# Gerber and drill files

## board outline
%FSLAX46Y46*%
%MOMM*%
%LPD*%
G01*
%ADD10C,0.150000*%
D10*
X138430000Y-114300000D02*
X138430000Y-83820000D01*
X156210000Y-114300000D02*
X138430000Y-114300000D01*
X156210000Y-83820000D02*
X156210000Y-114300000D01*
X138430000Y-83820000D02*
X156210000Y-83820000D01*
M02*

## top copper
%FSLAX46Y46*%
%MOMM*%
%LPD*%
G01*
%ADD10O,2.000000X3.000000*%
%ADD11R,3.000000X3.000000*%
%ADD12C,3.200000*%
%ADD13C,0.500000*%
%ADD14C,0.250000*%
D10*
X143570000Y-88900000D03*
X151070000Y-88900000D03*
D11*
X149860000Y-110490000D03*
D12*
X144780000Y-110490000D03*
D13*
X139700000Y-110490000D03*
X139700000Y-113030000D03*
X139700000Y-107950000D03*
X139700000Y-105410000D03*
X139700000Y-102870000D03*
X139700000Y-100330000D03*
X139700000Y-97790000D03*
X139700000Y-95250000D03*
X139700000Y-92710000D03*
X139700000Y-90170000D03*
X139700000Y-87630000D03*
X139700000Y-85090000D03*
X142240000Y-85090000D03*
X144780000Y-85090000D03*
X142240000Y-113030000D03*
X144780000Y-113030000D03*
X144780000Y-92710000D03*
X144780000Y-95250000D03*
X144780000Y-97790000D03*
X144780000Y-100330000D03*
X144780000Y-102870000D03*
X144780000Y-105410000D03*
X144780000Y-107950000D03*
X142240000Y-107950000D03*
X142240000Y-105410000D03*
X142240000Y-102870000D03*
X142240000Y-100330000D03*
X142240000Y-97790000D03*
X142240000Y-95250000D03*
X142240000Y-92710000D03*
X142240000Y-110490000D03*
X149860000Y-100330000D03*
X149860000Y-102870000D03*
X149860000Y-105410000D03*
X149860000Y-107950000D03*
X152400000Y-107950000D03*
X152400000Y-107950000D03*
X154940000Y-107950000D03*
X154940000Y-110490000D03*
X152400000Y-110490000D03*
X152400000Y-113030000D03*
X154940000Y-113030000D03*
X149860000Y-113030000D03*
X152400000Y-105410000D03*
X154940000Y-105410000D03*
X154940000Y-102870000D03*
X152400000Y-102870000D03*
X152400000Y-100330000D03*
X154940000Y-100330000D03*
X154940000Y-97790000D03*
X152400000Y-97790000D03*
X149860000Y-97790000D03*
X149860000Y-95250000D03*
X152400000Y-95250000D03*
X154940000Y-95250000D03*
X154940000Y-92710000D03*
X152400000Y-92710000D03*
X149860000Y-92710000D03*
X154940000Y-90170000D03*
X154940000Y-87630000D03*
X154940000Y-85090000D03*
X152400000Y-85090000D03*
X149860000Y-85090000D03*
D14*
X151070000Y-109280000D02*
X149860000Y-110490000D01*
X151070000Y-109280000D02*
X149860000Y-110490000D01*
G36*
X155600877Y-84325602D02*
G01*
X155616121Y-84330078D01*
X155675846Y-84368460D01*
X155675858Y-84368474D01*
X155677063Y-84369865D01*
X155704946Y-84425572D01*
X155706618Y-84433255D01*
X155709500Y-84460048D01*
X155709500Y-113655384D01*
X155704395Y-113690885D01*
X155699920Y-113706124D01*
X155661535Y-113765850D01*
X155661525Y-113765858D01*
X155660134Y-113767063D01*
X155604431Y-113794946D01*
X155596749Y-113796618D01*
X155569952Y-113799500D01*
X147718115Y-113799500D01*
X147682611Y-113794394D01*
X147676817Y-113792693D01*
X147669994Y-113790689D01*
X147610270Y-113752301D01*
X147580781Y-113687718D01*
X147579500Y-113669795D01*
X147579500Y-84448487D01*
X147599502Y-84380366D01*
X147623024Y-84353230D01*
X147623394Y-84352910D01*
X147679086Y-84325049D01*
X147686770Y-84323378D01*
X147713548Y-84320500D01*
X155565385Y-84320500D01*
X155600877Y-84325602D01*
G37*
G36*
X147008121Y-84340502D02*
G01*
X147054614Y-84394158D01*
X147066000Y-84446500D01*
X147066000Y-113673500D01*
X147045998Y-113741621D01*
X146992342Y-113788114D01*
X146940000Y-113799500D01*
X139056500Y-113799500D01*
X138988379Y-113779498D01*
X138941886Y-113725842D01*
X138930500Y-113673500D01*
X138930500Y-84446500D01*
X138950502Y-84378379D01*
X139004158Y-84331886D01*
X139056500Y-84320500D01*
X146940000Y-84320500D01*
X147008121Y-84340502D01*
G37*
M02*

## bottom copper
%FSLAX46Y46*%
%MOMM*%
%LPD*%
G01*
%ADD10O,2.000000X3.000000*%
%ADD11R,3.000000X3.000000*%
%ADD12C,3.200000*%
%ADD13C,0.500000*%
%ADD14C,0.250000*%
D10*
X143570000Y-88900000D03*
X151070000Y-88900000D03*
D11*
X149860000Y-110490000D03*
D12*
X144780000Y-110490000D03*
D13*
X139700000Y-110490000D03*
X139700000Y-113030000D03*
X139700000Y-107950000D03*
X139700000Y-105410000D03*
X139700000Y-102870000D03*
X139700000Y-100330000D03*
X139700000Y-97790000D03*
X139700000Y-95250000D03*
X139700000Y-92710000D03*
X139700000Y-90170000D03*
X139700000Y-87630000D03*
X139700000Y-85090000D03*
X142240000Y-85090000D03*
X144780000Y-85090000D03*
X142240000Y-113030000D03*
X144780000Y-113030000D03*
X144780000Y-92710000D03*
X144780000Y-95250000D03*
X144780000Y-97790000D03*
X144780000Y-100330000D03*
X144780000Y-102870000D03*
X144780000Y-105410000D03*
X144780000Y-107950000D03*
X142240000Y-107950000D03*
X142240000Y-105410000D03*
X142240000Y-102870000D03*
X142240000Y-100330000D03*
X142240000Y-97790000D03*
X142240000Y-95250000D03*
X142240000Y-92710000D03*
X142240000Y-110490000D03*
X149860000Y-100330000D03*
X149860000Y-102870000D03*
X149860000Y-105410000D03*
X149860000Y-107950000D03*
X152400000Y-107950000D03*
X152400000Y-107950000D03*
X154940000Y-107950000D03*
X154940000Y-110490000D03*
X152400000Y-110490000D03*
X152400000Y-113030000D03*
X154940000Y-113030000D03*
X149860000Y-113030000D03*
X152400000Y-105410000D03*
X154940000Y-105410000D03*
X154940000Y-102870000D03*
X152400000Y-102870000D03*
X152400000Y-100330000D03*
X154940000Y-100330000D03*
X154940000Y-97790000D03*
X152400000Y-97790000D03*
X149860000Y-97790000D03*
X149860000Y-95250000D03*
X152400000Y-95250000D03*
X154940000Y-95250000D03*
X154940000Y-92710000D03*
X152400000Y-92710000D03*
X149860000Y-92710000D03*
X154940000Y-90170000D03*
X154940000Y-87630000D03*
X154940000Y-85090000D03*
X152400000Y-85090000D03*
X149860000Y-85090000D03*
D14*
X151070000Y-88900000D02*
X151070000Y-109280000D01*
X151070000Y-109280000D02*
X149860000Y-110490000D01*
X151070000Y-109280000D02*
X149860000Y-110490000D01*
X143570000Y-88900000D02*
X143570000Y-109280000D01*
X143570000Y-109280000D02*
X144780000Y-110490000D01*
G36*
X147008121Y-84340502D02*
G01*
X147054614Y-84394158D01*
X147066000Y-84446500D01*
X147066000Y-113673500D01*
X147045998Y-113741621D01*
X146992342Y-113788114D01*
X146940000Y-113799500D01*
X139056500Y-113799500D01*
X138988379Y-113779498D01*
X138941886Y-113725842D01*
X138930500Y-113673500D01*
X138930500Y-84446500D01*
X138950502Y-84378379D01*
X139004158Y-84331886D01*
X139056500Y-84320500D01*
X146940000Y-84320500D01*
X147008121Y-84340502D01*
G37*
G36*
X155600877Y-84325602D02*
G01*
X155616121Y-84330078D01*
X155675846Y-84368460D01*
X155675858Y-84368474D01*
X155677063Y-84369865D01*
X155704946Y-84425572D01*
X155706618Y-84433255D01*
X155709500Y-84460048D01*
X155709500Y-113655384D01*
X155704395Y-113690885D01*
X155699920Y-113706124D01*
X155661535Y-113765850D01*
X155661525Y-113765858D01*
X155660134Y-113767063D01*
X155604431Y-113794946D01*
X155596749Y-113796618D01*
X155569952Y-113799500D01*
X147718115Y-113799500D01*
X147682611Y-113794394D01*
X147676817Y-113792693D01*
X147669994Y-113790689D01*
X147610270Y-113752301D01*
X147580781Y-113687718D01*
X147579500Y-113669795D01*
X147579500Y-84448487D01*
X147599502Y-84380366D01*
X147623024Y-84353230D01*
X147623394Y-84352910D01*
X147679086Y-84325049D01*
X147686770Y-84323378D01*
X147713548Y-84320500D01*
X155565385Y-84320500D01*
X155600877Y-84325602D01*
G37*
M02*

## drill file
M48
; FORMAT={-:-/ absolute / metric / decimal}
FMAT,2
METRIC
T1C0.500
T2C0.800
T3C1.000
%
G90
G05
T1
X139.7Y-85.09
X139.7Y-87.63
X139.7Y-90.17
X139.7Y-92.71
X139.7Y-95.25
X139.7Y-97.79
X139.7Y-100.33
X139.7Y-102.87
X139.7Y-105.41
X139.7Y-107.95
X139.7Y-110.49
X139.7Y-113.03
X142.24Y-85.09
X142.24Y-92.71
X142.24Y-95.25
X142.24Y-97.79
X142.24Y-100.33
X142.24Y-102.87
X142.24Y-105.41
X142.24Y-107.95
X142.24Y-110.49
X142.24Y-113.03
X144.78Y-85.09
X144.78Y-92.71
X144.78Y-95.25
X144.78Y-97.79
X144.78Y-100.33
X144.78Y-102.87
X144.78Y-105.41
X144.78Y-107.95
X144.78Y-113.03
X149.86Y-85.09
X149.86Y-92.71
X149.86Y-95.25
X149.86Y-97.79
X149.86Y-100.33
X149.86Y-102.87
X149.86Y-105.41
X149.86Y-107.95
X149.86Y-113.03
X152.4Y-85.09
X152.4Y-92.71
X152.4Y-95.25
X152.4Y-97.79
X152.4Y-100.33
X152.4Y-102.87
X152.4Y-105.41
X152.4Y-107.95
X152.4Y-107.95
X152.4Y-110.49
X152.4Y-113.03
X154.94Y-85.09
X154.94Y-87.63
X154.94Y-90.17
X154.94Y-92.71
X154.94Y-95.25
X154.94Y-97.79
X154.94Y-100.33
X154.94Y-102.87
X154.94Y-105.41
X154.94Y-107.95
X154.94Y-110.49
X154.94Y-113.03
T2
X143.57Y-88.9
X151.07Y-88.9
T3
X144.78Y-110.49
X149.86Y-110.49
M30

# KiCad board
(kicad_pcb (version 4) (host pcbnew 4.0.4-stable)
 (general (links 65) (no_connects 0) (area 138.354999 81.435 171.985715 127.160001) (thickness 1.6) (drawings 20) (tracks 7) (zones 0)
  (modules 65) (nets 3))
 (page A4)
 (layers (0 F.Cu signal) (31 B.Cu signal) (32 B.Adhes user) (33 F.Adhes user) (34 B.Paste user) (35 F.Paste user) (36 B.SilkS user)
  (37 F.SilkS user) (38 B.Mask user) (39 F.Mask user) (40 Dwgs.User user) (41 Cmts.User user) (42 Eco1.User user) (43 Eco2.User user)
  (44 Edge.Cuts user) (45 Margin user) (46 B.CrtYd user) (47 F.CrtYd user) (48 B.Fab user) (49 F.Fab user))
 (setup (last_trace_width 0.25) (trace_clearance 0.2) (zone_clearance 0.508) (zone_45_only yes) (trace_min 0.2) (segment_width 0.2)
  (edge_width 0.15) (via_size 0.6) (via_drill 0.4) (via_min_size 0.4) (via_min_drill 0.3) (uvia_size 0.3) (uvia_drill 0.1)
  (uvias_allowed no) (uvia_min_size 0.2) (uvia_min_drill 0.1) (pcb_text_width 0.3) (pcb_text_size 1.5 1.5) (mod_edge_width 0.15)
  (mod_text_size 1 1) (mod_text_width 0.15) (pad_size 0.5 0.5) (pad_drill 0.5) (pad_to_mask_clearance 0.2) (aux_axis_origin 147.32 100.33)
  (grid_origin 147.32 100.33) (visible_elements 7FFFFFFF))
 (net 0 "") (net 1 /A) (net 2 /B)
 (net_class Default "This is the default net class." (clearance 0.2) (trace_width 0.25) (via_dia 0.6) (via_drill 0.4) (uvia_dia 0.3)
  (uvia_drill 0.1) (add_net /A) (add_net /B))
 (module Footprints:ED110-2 (layer F.Cu) (at 147.32 88.9)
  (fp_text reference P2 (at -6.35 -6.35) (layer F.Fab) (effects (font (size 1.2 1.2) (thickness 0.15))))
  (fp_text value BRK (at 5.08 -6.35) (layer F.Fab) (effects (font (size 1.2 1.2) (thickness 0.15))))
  (pad 1 thru_hole oval (at -3.75 0) (size 2 3) (drill 0.8) (layers *.Cu *.Mask) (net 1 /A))
  (pad 2 thru_hole oval (at 3.75 0) (size 2 3) (drill 0.8) (layers *.Cu *.Mask) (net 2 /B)))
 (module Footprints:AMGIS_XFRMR (layer F.Cu) (at 147.32 110.49 180)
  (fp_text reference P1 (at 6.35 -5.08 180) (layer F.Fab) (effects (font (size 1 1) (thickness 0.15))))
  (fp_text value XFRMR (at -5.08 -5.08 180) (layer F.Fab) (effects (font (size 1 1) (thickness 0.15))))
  (pad 1 thru_hole rect (at -2.54 0 180) (size 3 3) (drill 1) (layers *.Cu *.Mask) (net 2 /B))
  (pad 2 thru_hole circle (at 2.54 0 180) (size 3.2 3.2) (drill 1) (layers *.Cu *.Mask) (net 1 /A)))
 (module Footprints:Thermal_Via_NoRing (layer F.Cu) (at 139.7 110.49)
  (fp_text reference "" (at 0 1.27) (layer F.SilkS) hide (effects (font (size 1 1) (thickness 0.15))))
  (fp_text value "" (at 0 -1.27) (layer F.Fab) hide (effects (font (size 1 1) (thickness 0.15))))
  (pad "" thru_hole circle (at 0 0) (size 0.5 0.5) (drill 0.5) (layers *.Cu *.Mask) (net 1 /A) (solder_mask_margin 0.01)))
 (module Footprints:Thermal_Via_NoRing (layer F.Cu) (at 139.7 113.03)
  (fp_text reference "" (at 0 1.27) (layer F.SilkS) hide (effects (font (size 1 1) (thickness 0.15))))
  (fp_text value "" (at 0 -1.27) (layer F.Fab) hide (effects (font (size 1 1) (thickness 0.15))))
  (pad "" thru_hole circle (at 0 0) (size 0.5 0.5) (drill 0.5) (layers *.Cu *.Mask) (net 1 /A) (solder_mask_margin 0.01)))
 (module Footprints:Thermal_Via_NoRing (layer F.Cu) (at 139.7 107.95)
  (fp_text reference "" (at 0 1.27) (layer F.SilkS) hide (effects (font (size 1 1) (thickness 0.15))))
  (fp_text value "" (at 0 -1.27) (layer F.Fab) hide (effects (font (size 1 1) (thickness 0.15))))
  (pad "" thru_hole circle (at 0 0) (size 0.5 0.5) (drill 0.5) (layers *.Cu *.Mask) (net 1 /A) (solder_mask_margin 0.01)))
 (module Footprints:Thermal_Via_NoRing (layer F.Cu) (at 139.7 105.41)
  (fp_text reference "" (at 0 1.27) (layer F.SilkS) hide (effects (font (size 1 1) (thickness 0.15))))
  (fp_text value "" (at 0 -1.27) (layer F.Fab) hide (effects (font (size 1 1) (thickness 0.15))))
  (pad "" thru_hole circle (at 0 0) (size 0.5 0.5) (drill 0.5) (layers *.Cu *.Mask) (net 1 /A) (solder_mask_margin 0.01)))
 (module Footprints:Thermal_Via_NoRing (layer F.Cu) (at 139.7 102.87)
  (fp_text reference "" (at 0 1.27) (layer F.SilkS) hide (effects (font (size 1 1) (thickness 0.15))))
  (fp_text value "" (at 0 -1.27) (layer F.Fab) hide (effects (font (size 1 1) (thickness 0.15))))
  (pad "" thru_hole circle (at 0 0) (size 0.5 0.5) (drill 0.5) (layers *.Cu *.Mask) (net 1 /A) (solder_mask_margin 0.01)))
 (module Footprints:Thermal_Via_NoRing (layer F.Cu) (at 139.7 100.33)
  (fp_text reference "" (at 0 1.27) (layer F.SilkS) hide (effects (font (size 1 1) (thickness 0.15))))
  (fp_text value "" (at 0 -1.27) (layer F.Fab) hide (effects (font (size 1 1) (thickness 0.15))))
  (pad "" thru_hole circle (at 0 0) (size 0.5 0.5) (drill 0.5) (layers *.Cu *.Mask) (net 1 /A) (solder_mask_margin 0.01)))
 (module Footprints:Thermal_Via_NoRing (layer F.Cu) (at 139.7 97.79)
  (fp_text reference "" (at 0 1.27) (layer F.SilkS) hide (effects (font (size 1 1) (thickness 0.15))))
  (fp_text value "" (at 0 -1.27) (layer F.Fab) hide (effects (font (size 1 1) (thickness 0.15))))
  (pad "" thru_hole circle (at 0 0) (size 0.5 0.5) (drill 0.5) (layers *.Cu *.Mask) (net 1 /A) (solder_mask_margin 0.01)))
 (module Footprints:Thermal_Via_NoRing (layer F.Cu) (at 139.7 95.25)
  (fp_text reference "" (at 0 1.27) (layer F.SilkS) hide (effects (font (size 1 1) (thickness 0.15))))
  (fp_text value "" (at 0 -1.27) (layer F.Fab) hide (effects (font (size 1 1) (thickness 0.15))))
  (pad "" thru_hole circle (at 0 0) (size 0.5 0.5) (drill 0.5) (layers *.Cu *.Mask) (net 1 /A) (solder_mask_margin 0.01)))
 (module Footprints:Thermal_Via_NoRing (layer F.Cu) (at 139.7 92.71)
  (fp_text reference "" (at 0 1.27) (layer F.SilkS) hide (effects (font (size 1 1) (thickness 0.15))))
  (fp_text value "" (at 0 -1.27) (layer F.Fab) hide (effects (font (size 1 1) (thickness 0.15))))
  (pad "" thru_hole circle (at 0 0) (size 0.5 0.5) (drill 0.5) (layers *.Cu *.Mask) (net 1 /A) (solder_mask_margin 0.01)))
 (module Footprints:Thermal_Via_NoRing (layer F.Cu) (at 139.7 90.17)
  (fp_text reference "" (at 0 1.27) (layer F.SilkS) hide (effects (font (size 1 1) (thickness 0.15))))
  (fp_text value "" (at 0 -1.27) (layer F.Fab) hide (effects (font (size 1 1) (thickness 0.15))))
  (pad "" thru_hole circle (at 0 0) (size 0.5 0.5) (drill 0.5) (layers *.Cu *.Mask) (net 1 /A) (solder_mask_margin 0.01)))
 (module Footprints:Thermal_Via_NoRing (layer F.Cu) (at 139.7 87.63)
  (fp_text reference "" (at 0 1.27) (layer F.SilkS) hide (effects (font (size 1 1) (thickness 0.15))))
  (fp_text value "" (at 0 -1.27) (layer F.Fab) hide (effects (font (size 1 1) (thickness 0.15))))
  (pad "" thru_hole circle (at 0 0) (size 0.5 0.5) (drill 0.5) (layers *.Cu *.Mask) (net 1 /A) (solder_mask_margin 0.01)))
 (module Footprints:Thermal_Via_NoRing (layer F.Cu) (at 139.7 85.09)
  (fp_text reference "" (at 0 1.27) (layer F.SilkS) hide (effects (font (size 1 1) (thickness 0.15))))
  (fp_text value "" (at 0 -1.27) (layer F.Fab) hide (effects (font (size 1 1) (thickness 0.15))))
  (pad "" thru_hole circle (at 0 0) (size 0.5 0.5) (drill 0.5) (layers *.Cu *.Mask) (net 1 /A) (solder_mask_margin 0.01)))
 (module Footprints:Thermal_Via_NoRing (layer F.Cu) (at 142.24 85.09)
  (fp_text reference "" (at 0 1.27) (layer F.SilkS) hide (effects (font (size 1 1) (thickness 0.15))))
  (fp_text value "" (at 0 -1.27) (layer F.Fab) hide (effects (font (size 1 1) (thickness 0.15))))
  (pad "" thru_hole circle (at 0 0) (size 0.5 0.5) (drill 0.5) (layers *.Cu *.Mask) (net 1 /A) (solder_mask_margin 0.01)))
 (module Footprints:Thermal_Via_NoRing (layer F.Cu) (at 144.78 85.09)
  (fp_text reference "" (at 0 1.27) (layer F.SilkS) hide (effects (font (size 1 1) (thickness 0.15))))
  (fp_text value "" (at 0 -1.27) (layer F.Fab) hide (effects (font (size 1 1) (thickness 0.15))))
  (pad "" thru_hole circle (at 0 0) (size 0.5 0.5) (drill 0.5) (layers *.Cu *.Mask) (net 1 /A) (solder_mask_margin 0.01)))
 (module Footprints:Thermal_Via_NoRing (layer F.Cu) (at 142.24 113.03)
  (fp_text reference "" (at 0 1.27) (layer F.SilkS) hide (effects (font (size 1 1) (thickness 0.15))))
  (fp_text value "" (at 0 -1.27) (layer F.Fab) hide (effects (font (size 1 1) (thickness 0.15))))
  (pad "" thru_hole circle (at 0 0) (size 0.5 0.5) (drill 0.5) (layers *.Cu *.Mask) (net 1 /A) (solder_mask_margin 0.01)))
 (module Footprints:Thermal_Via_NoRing (layer F.Cu) (at 144.78 113.03)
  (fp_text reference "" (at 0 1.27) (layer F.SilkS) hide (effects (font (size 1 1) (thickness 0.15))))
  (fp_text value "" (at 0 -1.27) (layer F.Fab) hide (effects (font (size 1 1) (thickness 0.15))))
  (pad "" thru_hole circle (at 0 0) (size 0.5 0.5) (drill 0.5) (layers *.Cu *.Mask) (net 1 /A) (solder_mask_margin 0.01)))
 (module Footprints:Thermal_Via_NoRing (layer F.Cu) (at 144.78 92.71)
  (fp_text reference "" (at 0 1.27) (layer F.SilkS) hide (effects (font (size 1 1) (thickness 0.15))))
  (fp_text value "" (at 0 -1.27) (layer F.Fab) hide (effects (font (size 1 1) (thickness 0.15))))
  (pad "" thru_hole circle (at 0 0) (size 0.5 0.5) (drill 0.5) (layers *.Cu *.Mask) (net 1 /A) (solder_mask_margin 0.01)))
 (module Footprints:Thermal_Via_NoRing (layer F.Cu) (at 144.78 95.25)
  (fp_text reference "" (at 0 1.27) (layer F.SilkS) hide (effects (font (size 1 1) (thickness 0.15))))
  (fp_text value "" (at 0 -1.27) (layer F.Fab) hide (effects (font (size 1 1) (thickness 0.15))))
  (pad "" thru_hole circle (at 0 0) (size 0.5 0.5) (drill 0.5) (layers *.Cu *.Mask) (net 1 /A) (solder_mask_margin 0.01)))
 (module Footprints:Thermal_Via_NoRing (layer F.Cu) (at 144.78 97.79)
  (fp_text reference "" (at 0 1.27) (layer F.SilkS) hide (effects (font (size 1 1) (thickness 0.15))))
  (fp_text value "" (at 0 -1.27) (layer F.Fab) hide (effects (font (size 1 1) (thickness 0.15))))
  (pad "" thru_hole circle (at 0 0) (size 0.5 0.5) (drill 0.5) (layers *.Cu *.Mask) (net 1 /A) (solder_mask_margin 0.01)))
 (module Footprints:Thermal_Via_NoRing (layer F.Cu) (at 144.78 100.33)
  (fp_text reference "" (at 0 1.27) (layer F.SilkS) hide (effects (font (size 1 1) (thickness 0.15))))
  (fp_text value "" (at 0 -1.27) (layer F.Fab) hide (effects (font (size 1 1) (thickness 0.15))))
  (pad "" thru_hole circle (at 0 0) (size 0.5 0.5) (drill 0.5) (layers *.Cu *.Mask) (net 1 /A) (solder_mask_margin 0.01)))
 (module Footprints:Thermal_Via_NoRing (layer F.Cu) (at 144.78 102.87)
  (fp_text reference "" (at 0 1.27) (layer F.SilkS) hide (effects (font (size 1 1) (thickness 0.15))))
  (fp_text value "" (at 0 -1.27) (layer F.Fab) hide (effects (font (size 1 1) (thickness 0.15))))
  (pad "" thru_hole circle (at 0 0) (size 0.5 0.5) (drill 0.5) (layers *.Cu *.Mask) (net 1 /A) (solder_mask_margin 0.01)))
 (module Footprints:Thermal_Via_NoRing (layer F.Cu) (at 144.78 105.41)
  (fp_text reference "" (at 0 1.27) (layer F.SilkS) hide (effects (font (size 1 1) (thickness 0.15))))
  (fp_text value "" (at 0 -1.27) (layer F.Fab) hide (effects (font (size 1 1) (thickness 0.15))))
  (pad "" thru_hole circle (at 0 0) (size 0.5 0.5) (drill 0.5) (layers *.Cu *.Mask) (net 1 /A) (solder_mask_margin 0.01)))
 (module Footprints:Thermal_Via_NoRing (layer F.Cu) (at 144.78 107.95)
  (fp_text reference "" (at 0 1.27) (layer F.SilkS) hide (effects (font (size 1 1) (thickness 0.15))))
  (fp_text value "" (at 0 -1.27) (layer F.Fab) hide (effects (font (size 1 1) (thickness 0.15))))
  (pad "" thru_hole circle (at 0 0) (size 0.5 0.5) (drill 0.5) (layers *.Cu *.Mask) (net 1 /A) (solder_mask_margin 0.01)))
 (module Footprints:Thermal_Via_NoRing (layer F.Cu) (at 142.24 107.95)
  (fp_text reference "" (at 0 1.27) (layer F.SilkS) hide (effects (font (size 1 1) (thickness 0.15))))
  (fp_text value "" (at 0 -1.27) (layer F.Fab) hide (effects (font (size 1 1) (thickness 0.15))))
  (pad "" thru_hole circle (at 0 0) (size 0.5 0.5) (drill 0.5) (layers *.Cu *.Mask) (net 1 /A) (solder_mask_margin 0.01)))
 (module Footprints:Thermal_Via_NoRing (layer F.Cu) (at 142.24 105.41)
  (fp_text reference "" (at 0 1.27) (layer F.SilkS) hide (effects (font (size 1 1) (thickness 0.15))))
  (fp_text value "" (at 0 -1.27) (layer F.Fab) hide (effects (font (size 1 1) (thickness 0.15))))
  (pad "" thru_hole circle (at 0 0) (size 0.5 0.5) (drill 0.5) (layers *.Cu *.Mask) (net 1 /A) (solder_mask_margin 0.01)))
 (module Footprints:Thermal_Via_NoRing (layer F.Cu) (at 142.24 102.87)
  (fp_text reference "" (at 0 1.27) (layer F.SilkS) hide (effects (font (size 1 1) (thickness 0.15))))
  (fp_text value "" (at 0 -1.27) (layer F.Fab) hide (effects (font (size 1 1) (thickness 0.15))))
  (pad "" thru_hole circle (at 0 0) (size 0.5 0.5) (drill 0.5) (layers *.Cu *.Mask) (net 1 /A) (solder_mask_margin 0.01)))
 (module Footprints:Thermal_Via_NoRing (layer F.Cu) (at 142.24 100.33)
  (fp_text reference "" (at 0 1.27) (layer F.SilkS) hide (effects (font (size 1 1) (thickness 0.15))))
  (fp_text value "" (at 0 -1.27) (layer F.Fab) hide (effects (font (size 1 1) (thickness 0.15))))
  (pad "" thru_hole circle (at 0 0) (size 0.5 0.5) (drill 0.5) (layers *.Cu *.Mask) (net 1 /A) (solder_mask_margin 0.01)))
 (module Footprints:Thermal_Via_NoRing (layer F.Cu) (at 142.24 97.79)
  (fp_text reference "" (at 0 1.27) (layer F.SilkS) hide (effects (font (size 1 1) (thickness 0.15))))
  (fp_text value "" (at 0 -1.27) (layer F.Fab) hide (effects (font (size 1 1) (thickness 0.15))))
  (pad "" thru_hole circle (at 0 0) (size 0.5 0.5) (drill 0.5) (layers *.Cu *.Mask) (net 1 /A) (solder_mask_margin 0.01)))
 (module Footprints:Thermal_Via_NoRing (layer F.Cu) (at 142.24 95.25)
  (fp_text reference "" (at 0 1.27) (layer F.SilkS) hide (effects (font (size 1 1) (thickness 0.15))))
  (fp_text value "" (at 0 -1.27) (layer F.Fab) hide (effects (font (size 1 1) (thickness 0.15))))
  (pad "" thru_hole circle (at 0 0) (size 0.5 0.5) (drill 0.5) (layers *.Cu *.Mask) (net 1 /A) (solder_mask_margin 0.01)))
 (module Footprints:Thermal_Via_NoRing (layer F.Cu) (at 142.24 92.71)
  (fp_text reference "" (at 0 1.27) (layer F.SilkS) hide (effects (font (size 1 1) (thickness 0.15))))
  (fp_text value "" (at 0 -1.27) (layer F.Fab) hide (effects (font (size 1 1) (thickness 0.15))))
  (pad "" thru_hole circle (at 0 0) (size 0.5 0.5) (drill 0.5) (layers *.Cu *.Mask) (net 1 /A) (solder_mask_margin 0.01)))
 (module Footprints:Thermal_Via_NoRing (layer F.Cu) (at 142.24 110.49)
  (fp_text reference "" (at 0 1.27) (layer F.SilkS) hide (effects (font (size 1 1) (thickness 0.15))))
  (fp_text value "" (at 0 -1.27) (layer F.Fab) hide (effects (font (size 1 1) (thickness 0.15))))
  (pad "" thru_hole circle (at 0 0) (size 0.5 0.5) (drill 0.5) (layers *.Cu *.Mask) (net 1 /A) (solder_mask_margin 0.01)))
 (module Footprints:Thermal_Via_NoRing (layer F.Cu) (at 149.86 100.33)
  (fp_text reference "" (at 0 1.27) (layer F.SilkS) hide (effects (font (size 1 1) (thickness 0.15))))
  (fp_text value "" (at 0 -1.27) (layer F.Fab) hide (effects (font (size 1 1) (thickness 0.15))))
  (pad "" thru_hole circle (at 0 0) (size 0.5 0.5) (drill 0.5) (layers *.Cu *.Mask) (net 2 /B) (solder_mask_margin 0.01)))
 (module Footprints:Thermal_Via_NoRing (layer F.Cu) (at 149.86 102.87)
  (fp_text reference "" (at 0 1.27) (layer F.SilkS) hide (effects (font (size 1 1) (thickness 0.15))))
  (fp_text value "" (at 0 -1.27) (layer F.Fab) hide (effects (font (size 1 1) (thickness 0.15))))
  (pad "" thru_hole circle (at 0 0) (size 0.5 0.5) (drill 0.5) (layers *.Cu *.Mask) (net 2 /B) (solder_mask_margin 0.01)))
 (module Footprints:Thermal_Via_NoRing (layer F.Cu) (at 149.86 105.41)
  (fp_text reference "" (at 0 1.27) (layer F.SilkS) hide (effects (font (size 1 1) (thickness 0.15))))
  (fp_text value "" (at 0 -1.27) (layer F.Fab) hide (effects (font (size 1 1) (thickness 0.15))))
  (pad "" thru_hole circle (at 0 0) (size 0.5 0.5) (drill 0.5) (layers *.Cu *.Mask) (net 2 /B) (solder_mask_margin 0.01)))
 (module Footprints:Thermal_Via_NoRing (layer F.Cu) (at 149.86 107.95)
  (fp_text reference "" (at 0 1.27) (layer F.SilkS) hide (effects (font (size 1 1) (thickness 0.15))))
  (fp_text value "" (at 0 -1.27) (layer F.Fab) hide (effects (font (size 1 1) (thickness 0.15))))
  (pad "" thru_hole circle (at 0 0) (size 0.5 0.5) (drill 0.5) (layers *.Cu *.Mask) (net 2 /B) (solder_mask_margin 0.01)))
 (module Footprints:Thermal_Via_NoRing (layer F.Cu) (at 152.4 107.95)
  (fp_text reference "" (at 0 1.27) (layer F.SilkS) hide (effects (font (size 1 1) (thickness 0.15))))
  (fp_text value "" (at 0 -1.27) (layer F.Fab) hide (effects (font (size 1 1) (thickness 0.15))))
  (pad "" thru_hole circle (at 0 0) (size 0.5 0.5) (drill 0.5) (layers *.Cu *.Mask) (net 2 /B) (solder_mask_margin 0.01)))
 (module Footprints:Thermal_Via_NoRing (layer F.Cu) (at 152.4 107.95)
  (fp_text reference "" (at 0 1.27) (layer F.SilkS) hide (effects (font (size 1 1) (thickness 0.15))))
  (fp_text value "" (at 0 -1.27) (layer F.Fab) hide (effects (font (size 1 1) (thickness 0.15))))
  (pad "" thru_hole circle (at 0 0) (size 0.5 0.5) (drill 0.5) (layers *.Cu *.Mask) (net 2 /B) (solder_mask_margin 0.01)))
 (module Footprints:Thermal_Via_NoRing (layer F.Cu) (at 154.94 107.95)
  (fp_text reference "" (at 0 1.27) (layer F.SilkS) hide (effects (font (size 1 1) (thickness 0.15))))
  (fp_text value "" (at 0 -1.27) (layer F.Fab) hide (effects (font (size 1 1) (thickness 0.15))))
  (pad "" thru_hole circle (at 0 0) (size 0.5 0.5) (drill 0.5) (layers *.Cu *.Mask) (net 2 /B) (solder_mask_margin 0.01)))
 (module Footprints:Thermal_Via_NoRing (layer F.Cu) (at 154.94 110.49)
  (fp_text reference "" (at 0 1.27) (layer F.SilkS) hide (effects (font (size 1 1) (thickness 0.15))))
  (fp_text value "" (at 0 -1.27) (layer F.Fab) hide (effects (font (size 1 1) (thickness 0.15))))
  (pad "" thru_hole circle (at 0 0) (size 0.5 0.5) (drill 0.5) (layers *.Cu *.Mask) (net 2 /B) (solder_mask_margin 0.01)))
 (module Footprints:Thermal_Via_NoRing (layer F.Cu) (at 152.4 110.49)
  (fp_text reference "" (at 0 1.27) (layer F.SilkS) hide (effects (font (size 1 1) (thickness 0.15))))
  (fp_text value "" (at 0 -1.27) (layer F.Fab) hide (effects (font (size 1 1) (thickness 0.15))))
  (pad "" thru_hole circle (at 0 0) (size 0.5 0.5) (drill 0.5) (layers *.Cu *.Mask) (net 2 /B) (solder_mask_margin 0.01)))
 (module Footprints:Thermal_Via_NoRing (layer F.Cu) (at 152.4 113.03)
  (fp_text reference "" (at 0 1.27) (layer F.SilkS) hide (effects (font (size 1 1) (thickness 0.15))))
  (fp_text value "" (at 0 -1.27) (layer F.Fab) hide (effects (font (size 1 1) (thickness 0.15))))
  (pad "" thru_hole circle (at 0 0) (size 0.5 0.5) (drill 0.5) (layers *.Cu *.Mask) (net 2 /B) (solder_mask_margin 0.01)))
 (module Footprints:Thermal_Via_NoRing (layer F.Cu) (at 154.94 113.03)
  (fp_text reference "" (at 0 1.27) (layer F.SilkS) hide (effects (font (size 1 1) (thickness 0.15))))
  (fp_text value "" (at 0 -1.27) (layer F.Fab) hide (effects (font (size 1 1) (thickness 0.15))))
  (pad "" thru_hole circle (at 0 0) (size 0.5 0.5) (drill 0.5) (layers *.Cu *.Mask) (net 2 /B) (solder_mask_margin 0.01)))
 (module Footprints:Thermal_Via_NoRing (layer F.Cu) (at 149.86 113.03)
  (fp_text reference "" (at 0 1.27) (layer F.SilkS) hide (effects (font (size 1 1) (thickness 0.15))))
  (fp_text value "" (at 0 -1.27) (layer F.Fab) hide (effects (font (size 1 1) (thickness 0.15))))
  (pad "" thru_hole circle (at 0 0) (size 0.5 0.5) (drill 0.5) (layers *.Cu *.Mask) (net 2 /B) (solder_mask_margin 0.01)))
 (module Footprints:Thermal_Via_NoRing (layer F.Cu) (at 152.4 105.41)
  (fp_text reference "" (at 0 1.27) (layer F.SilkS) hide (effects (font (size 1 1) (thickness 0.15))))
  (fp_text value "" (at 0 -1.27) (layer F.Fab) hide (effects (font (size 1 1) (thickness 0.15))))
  (pad "" thru_hole circle (at 0 0) (size 0.5 0.5) (drill 0.5) (layers *.Cu *.Mask) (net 2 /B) (solder_mask_margin 0.01)))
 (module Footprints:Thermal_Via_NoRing (layer F.Cu) (at 154.94 105.41)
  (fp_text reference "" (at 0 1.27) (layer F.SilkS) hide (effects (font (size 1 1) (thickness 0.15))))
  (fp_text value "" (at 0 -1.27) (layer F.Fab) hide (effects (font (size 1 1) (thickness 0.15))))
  (pad "" thru_hole circle (at 0 0) (size 0.5 0.5) (drill 0.5) (layers *.Cu *.Mask) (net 2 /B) (solder_mask_margin 0.01)))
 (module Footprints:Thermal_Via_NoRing (layer F.Cu) (at 154.94 102.87)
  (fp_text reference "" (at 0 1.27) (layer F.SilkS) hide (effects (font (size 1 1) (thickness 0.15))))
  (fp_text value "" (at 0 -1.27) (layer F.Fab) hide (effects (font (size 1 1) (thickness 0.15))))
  (pad "" thru_hole circle (at 0 0) (size 0.5 0.5) (drill 0.5) (layers *.Cu *.Mask) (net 2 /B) (solder_mask_margin 0.01)))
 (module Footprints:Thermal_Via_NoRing (layer F.Cu) (at 152.4 102.87)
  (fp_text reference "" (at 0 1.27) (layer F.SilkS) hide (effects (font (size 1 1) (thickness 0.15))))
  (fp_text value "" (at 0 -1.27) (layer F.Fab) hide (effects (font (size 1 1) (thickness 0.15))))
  (pad "" thru_hole circle (at 0 0) (size 0.5 0.5) (drill 0.5) (layers *.Cu *.Mask) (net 2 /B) (solder_mask_margin 0.01)))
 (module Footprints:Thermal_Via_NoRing (layer F.Cu) (at 152.4 100.33)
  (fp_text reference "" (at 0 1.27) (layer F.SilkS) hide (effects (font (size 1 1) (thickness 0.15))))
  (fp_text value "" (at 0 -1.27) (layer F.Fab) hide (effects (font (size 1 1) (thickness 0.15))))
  (pad "" thru_hole circle (at 0 0) (size 0.5 0.5) (drill 0.5) (layers *.Cu *.Mask) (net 2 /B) (solder_mask_margin 0.01)))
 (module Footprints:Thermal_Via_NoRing (layer F.Cu) (at 154.94 100.33)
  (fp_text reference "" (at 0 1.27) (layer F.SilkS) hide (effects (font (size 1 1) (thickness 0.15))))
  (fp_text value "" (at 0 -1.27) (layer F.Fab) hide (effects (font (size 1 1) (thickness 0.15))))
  (pad "" thru_hole circle (at 0 0) (size 0.5 0.5) (drill 0.5) (layers *.Cu *.Mask) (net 2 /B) (solder_mask_margin 0.01)))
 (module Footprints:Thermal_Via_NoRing (layer F.Cu) (at 154.94 97.79)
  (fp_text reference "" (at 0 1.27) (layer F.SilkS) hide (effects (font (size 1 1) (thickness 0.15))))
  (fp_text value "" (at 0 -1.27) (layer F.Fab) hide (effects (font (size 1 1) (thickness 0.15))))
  (pad "" thru_hole circle (at 0 0) (size 0.5 0.5) (drill 0.5) (layers *.Cu *.Mask) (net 2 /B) (solder_mask_margin 0.01)))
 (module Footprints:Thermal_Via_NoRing (layer F.Cu) (at 152.4 97.79)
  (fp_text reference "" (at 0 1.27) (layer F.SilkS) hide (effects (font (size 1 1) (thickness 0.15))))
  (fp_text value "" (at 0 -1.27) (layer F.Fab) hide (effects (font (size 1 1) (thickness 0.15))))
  (pad "" thru_hole circle (at 0 0) (size 0.5 0.5) (drill 0.5) (layers *.Cu *.Mask) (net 2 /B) (solder_mask_margin 0.01)))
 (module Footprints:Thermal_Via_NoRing (layer F.Cu) (at 149.86 97.79)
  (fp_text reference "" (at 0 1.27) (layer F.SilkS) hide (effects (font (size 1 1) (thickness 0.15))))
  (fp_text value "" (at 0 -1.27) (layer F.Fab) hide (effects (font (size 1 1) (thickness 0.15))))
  (pad "" thru_hole circle (at 0 0) (size 0.5 0.5) (drill 0.5) (layers *.Cu *.Mask) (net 2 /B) (solder_mask_margin 0.01)))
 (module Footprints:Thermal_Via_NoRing (layer F.Cu) (at 149.86 95.25)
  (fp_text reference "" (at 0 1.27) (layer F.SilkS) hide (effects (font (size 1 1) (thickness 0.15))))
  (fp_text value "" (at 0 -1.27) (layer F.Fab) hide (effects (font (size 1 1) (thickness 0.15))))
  (pad "" thru_hole circle (at 0 0) (size 0.5 0.5) (drill 0.5) (layers *.Cu *.Mask) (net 2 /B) (solder_mask_margin 0.01)))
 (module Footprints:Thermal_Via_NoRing (layer F.Cu) (at 152.4 95.25)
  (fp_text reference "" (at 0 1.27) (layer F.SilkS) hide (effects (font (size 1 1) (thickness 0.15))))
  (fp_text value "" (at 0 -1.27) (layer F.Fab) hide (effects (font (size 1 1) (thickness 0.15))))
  (pad "" thru_hole circle (at 0 0) (size 0.5 0.5) (drill 0.5) (layers *.Cu *.Mask) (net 2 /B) (solder_mask_margin 0.01)))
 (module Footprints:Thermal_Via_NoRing (layer F.Cu) (at 154.94 95.25)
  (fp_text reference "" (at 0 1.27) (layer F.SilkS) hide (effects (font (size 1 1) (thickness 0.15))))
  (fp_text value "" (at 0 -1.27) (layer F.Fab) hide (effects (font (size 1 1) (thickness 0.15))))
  (pad "" thru_hole circle (at 0 0) (size 0.5 0.5) (drill 0.5) (layers *.Cu *.Mask) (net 2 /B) (solder_mask_margin 0.01)))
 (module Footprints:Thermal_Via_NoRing (layer F.Cu) (at 154.94 92.71)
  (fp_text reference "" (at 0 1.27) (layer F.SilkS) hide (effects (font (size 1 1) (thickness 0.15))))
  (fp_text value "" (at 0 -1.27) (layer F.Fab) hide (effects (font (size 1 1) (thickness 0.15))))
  (pad "" thru_hole circle (at 0 0) (size 0.5 0.5) (drill 0.5) (layers *.Cu *.Mask) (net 2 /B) (solder_mask_margin 0.01)))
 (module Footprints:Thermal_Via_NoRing (layer F.Cu) (at 152.4 92.71)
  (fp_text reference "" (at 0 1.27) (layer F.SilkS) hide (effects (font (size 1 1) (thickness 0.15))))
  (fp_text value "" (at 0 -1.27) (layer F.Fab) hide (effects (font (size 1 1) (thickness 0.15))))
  (pad "" thru_hole circle (at 0 0) (size 0.5 0.5) (drill 0.5) (layers *.Cu *.Mask) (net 2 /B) (solder_mask_margin 0.01)))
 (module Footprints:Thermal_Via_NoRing (layer F.Cu) (at 149.86 92.71)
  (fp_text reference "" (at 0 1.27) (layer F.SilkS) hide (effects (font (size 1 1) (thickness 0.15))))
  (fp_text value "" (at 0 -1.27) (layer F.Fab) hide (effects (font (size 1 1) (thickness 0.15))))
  (pad "" thru_hole circle (at 0 0) (size 0.5 0.5) (drill 0.5) (layers *.Cu *.Mask) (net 2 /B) (solder_mask_margin 0.01)))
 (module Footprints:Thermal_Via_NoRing (layer F.Cu) (at 154.94 90.17)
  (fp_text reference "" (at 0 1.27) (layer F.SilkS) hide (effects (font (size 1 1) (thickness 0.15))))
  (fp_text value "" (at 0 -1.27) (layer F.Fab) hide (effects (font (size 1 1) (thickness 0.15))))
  (pad "" thru_hole circle (at 0 0) (size 0.5 0.5) (drill 0.5) (layers *.Cu *.Mask) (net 2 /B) (solder_mask_margin 0.01)))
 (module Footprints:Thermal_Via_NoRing (layer F.Cu) (at 154.94 87.63)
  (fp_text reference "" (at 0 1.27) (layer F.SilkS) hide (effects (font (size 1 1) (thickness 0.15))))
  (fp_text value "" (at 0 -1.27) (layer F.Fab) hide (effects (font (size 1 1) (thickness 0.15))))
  (pad "" thru_hole circle (at 0 0) (size 0.5 0.5) (drill 0.5) (layers *.Cu *.Mask) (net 2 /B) (solder_mask_margin 0.01)))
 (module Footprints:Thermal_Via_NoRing (layer F.Cu) (at 154.94 85.09)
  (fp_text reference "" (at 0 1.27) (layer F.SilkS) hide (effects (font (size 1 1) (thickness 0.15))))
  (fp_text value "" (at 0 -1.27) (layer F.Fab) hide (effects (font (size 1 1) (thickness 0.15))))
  (pad "" thru_hole circle (at 0 0) (size 0.5 0.5) (drill 0.5) (layers *.Cu *.Mask) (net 2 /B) (solder_mask_margin 0.01)))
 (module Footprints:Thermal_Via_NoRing (layer F.Cu) (at 152.4 85.09)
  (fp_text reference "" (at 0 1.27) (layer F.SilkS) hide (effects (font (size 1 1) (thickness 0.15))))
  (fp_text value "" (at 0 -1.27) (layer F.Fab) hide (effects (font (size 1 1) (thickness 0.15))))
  (pad "" thru_hole circle (at 0 0) (size 0.5 0.5) (drill 0.5) (layers *.Cu *.Mask) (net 2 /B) (solder_mask_margin 0.01)))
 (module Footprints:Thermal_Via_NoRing (layer F.Cu) (at 149.86 85.09)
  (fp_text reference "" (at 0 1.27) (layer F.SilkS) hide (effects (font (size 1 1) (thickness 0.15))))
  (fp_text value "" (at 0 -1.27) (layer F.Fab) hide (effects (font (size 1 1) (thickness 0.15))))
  (pad "" thru_hole circle (at 0 0) (size 0.5 0.5) (drill 0.5) (layers *.Cu *.Mask) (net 2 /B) (solder_mask_margin 0.01)))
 (gr_line (start 138.43 114.3) (end 138.43 83.82) (angle 90) (layer Edge.Cuts) (width 0.15))
 (gr_line (start 156.21 114.3) (end 138.43 114.3) (angle 90) (layer Edge.Cuts) (width 0.15))
 (gr_line (start 156.21 83.82) (end 156.21 114.3) (angle 90) (layer Edge.Cuts) (width 0.15))
 (gr_line (start 138.43 83.82) (end 156.21 83.82) (angle 90) (layer Edge.Cuts) (width 0.15))
 (segment (start 151.07 88.9) (end 151.07 109.28) (width 0.25) (layer B.Cu) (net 2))
 (segment (start 151.07 109.28) (end 149.86 110.49) (width 0.25) (layer B.Cu) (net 2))
 (segment (start 151.07 109.28) (end 149.86 110.49) (width 0.25) (layer F.Cu) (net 2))
 (segment (start 151.07 109.28) (end 149.86 110.49) (width 0.25) (layer B.Cu) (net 2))
 (segment (start 151.07 109.28) (end 149.86 110.49) (width 0.25) (layer F.Cu) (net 2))
 (segment (start 143.57 88.9) (end 143.57 109.28) (width 0.25) (layer B.Cu) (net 1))
 (segment (start 143.57 109.28) (end 144.78 110.49) (width 0.25) (layer B.Cu) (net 1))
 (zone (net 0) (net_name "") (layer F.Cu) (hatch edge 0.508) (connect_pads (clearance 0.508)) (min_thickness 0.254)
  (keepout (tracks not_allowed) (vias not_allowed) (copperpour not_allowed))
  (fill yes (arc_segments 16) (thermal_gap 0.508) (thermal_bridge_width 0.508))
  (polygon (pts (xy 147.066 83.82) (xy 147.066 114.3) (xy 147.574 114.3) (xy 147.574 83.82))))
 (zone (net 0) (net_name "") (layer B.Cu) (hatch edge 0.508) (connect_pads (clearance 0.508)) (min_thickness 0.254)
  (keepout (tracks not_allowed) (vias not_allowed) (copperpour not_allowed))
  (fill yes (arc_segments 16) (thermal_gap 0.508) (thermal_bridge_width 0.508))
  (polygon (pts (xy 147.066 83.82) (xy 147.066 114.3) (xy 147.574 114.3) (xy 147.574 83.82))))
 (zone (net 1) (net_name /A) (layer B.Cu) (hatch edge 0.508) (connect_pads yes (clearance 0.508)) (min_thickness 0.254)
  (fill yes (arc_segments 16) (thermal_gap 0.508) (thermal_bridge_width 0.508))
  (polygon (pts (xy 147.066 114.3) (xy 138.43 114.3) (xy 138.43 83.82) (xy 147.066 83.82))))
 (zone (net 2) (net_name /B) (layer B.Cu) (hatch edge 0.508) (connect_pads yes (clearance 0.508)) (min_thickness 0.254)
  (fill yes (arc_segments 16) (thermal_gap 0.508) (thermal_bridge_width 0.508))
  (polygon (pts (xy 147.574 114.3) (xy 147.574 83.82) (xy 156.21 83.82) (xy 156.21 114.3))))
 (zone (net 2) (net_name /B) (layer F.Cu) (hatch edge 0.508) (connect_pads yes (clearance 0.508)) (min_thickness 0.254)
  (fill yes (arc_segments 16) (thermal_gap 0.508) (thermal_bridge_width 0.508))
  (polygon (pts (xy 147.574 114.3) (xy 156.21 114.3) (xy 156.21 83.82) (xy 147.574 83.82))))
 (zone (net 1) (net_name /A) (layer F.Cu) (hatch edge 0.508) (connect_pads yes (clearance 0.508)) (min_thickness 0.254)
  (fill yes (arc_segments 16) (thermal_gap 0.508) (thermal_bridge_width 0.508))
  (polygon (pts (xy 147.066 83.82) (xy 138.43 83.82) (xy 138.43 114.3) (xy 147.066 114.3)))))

